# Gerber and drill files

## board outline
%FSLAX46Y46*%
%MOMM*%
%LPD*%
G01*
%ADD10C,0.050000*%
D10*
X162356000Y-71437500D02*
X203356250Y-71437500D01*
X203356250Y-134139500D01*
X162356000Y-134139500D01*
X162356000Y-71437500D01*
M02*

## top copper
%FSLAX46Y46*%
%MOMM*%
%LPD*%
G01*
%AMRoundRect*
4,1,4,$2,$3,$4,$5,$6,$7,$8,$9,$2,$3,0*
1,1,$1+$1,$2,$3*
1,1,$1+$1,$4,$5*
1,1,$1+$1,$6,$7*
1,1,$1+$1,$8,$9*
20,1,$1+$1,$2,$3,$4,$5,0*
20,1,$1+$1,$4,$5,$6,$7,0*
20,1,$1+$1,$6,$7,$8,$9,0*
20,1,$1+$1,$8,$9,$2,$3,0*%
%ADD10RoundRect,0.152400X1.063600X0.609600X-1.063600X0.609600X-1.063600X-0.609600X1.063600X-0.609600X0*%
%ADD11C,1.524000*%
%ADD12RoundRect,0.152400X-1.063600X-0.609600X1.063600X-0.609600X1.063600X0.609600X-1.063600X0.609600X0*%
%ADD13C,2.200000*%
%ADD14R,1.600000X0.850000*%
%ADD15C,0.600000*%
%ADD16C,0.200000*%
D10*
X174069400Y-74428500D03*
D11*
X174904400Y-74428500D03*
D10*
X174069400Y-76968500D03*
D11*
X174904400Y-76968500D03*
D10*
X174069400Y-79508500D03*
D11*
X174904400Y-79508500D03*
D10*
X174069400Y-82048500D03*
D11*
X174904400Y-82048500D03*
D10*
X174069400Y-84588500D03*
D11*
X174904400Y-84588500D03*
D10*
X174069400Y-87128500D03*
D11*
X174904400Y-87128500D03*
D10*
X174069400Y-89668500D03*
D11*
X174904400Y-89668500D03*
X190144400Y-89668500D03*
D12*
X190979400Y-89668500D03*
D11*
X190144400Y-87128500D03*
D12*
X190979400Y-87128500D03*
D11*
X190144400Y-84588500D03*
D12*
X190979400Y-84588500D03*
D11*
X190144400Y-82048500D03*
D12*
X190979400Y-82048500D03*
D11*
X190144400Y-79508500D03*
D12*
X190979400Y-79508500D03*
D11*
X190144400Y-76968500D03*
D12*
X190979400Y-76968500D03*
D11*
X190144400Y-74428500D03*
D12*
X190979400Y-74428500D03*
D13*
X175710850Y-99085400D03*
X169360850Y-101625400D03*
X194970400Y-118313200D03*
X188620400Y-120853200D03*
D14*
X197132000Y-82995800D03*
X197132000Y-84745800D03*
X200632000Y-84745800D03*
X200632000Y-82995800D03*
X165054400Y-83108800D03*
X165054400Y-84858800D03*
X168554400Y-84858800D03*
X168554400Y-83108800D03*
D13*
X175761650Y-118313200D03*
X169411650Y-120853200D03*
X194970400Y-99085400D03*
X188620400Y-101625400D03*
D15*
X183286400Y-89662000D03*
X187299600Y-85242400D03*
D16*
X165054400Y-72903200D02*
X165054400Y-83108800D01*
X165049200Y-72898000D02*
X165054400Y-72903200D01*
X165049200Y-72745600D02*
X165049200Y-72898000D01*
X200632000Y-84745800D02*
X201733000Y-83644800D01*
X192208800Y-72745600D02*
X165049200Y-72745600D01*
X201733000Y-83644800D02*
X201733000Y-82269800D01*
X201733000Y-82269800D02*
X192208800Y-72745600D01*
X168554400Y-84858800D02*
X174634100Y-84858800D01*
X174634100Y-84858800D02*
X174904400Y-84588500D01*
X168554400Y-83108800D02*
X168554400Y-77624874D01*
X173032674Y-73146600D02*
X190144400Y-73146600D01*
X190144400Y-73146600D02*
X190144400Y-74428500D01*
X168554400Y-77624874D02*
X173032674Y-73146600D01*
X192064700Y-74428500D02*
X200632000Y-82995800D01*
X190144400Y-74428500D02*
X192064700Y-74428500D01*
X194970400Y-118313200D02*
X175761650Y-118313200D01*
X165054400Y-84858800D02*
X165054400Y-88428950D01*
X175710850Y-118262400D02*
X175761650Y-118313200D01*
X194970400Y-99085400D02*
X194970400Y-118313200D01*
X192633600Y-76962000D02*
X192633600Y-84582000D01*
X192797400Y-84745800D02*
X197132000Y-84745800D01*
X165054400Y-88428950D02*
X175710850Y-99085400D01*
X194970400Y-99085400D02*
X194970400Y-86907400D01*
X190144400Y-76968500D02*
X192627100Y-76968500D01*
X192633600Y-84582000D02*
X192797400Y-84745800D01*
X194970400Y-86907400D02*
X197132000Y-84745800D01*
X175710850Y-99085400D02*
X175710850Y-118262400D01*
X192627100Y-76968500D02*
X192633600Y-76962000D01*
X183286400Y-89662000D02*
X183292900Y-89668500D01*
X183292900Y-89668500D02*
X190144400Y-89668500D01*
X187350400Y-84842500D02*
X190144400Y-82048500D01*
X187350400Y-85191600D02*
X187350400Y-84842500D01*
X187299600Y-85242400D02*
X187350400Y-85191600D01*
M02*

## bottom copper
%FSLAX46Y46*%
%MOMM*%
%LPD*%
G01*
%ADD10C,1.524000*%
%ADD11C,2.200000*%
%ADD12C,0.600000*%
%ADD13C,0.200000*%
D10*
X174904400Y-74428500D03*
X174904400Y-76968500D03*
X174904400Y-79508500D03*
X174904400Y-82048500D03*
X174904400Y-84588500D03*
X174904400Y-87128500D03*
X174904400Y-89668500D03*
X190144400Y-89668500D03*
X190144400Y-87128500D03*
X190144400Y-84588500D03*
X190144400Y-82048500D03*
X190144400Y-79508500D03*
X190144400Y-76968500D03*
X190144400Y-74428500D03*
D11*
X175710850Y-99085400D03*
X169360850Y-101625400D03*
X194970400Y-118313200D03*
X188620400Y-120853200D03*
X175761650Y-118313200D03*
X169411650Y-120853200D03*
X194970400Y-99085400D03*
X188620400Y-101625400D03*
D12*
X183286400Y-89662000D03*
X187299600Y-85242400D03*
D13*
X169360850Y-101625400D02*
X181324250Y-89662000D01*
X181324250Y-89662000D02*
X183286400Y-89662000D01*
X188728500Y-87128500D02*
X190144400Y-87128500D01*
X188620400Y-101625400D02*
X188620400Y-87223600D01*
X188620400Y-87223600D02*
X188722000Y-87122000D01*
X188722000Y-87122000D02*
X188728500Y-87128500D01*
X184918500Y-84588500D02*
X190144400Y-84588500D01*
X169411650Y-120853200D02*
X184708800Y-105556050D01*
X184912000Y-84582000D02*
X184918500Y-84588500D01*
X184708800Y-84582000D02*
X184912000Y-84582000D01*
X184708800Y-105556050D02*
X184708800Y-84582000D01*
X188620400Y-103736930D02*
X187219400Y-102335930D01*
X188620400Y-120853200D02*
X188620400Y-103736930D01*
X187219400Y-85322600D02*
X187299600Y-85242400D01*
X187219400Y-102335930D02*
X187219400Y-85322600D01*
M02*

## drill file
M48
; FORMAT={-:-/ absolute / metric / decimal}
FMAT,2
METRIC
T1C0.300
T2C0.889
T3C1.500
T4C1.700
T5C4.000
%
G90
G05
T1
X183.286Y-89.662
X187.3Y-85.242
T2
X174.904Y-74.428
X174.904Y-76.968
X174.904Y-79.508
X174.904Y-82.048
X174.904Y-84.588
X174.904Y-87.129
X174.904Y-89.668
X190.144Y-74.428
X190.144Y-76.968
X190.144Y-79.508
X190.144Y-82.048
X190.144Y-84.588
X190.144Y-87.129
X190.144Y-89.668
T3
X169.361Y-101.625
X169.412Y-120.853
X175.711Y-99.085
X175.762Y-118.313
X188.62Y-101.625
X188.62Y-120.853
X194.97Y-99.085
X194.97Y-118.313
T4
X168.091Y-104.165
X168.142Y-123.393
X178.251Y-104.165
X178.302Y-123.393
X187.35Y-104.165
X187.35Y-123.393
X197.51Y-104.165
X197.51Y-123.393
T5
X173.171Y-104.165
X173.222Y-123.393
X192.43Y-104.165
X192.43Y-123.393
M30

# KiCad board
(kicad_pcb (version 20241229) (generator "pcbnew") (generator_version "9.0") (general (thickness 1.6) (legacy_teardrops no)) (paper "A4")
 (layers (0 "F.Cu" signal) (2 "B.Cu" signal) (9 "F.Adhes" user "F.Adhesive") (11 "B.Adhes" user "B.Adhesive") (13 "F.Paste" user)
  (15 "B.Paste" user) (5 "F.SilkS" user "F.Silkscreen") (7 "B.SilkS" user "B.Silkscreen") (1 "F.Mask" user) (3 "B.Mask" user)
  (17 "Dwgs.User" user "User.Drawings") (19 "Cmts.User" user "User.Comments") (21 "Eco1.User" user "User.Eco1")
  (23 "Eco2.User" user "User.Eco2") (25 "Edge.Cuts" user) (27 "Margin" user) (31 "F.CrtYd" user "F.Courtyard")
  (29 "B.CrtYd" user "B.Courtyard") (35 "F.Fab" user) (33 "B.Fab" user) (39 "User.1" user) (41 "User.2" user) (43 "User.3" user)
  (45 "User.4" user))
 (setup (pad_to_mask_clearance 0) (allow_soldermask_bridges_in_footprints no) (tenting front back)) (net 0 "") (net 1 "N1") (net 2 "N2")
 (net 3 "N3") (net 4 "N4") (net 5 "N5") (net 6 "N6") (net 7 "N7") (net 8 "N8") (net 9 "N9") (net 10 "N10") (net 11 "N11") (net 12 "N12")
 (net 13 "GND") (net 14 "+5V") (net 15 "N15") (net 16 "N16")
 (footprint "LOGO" (layer "F.Cu") (at 199.6948 74.5236)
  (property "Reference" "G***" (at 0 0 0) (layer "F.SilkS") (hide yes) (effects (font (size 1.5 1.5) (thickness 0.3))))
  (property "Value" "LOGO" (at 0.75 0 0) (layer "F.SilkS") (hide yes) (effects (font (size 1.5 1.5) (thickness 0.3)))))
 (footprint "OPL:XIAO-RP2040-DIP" (layer "F.Cu") (at 182.5244 82.0485)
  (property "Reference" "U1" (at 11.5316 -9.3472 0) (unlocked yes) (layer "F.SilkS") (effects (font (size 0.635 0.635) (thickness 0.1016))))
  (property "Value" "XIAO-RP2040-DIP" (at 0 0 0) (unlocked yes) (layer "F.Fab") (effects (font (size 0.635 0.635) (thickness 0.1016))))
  (pad "1" smd roundrect (at -8.455 -7.62 180) (size 2.432 1.524) (layers "F.Cu" "F.Mask") (roundrect_rratio 0.1) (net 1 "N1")
   (thermal_bridge_angle 45))
  (pad "1" thru_hole circle (at -7.62 -7.62 180) (size 1.524 1.524) (drill 0.889) (layers "*.Cu" "*.Mask") (remove_unused_layers no)
   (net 1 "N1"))
  (pad "2" smd roundrect (at -8.455 -5.08 180) (size 2.432 1.524) (layers "F.Cu" "F.Mask") (roundrect_rratio 0.1) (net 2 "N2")
   (thermal_bridge_angle 45))
  (pad "2" thru_hole circle (at -7.62 -5.08 180) (size 1.524 1.524) (drill 0.889) (layers "*.Cu" "*.Mask") (remove_unused_layers no)
   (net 2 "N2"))
  (pad "3" smd roundrect (at -8.455 -2.54 180) (size 2.432 1.524) (layers "F.Cu" "F.Mask") (roundrect_rratio 0.1) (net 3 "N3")
   (thermal_bridge_angle 45))
  (pad "3" thru_hole circle (at -7.62 -2.54 180) (size 1.524 1.524) (drill 0.889) (layers "*.Cu" "*.Mask") (remove_unused_layers no)
   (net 3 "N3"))
  (pad "4" smd roundrect (at -8.455 0 180) (size 2.432 1.524) (layers "F.Cu" "F.Mask") (roundrect_rratio 0.1) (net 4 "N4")
   (thermal_bridge_angle 45))
  (pad "4" thru_hole circle (at -7.62 0 180) (size 1.524 1.524) (drill 0.889) (layers "*.Cu" "*.Mask") (remove_unused_layers no)
   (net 4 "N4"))
  (pad "5" smd roundrect (at -8.455 2.54 180) (size 2.432 1.524) (layers "F.Cu" "F.Mask") (roundrect_rratio 0.1) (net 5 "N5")
   (thermal_bridge_angle 45))
  (pad "5" thru_hole circle (at -7.62 2.54 180) (size 1.524 1.524) (drill 0.889) (layers "*.Cu" "*.Mask") (remove_unused_layers no)
   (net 5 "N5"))
  (pad "6" smd roundrect (at -8.455 5.08 180) (size 2.432 1.524) (layers "F.Cu" "F.Mask") (roundrect_rratio 0.1) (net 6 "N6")
   (thermal_bridge_angle 45))
  (pad "6" thru_hole circle (at -7.62 5.08 180) (size 1.524 1.524) (drill 0.889) (layers "*.Cu" "*.Mask") (remove_unused_layers no)
   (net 6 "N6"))
  (pad "7" smd roundrect (at -8.455 7.62 180) (size 2.432 1.524) (layers "F.Cu" "F.Mask") (roundrect_rratio 0.1) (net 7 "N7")
   (thermal_bridge_angle 45))
  (pad "7" thru_hole circle (at -7.62 7.62 180) (size 1.524 1.524) (drill 0.889) (layers "*.Cu" "*.Mask") (remove_unused_layers no)
   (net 7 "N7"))
  (pad "8" thru_hole circle (at 7.62 7.62) (size 1.524 1.524) (drill 0.889) (layers "*.Cu" "*.Mask") (remove_unused_layers no) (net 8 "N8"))
  (pad "8" smd roundrect (at 8.455 7.62) (size 2.432 1.524) (layers "F.Cu" "F.Mask") (roundrect_rratio 0.1) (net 8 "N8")
   (thermal_bridge_angle 45))
  (pad "9" thru_hole circle (at 7.62 5.08) (size 1.524 1.524) (drill 0.889) (layers "*.Cu" "*.Mask") (remove_unused_layers no) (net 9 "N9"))
  (pad "9" smd roundrect (at 8.455 5.08) (size 2.432 1.524) (layers "F.Cu" "F.Mask") (roundrect_rratio 0.1) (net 9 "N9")
   (thermal_bridge_angle 45))
  (pad "10" thru_hole circle (at 7.62 2.54) (size 1.524 1.524) (drill 0.889) (layers "*.Cu" "*.Mask") (remove_unused_layers no)
   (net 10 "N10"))
  (pad "10" smd roundrect (at 8.455 2.54) (size 2.432 1.524) (layers "F.Cu" "F.Mask") (roundrect_rratio 0.1) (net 10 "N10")
   (thermal_bridge_angle 45))
  (pad "11" thru_hole circle (at 7.62 0) (size 1.524 1.524) (drill 0.889) (layers "*.Cu" "*.Mask") (remove_unused_layers no) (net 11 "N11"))
  (pad "11" smd roundrect (at 8.455 0) (size 2.432 1.524) (layers "F.Cu" "F.Mask") (roundrect_rratio 0.1) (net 11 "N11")
   (thermal_bridge_angle 45))
  (pad "12" thru_hole circle (at 7.62 -2.54) (size 1.524 1.524) (drill 0.889) (layers "*.Cu" "*.Mask") (remove_unused_layers no)
   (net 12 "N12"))
  (pad "12" smd roundrect (at 8.455 -2.54) (size 2.432 1.524) (layers "F.Cu" "F.Mask") (roundrect_rratio 0.1) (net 12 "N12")
   (thermal_bridge_angle 45))
  (pad "13" thru_hole circle (at 7.62 -5.08) (size 1.524 1.524) (drill 0.889) (layers "*.Cu" "*.Mask") (remove_unused_layers no)
   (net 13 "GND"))
  (pad "13" smd roundrect (at 8.455 -5.08) (size 2.432 1.524) (layers "F.Cu" "F.Mask") (roundrect_rratio 0.1) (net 13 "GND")
   (thermal_bridge_angle 45))
  (pad "14" thru_hole circle (at 7.62 -7.62) (size 1.524 1.524) (drill 0.889) (layers "*.Cu" "*.Mask") (remove_unused_layers no)
   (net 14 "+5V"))
  (pad "14" smd roundrect (at 8.455 -7.62) (size 2.432 1.524) (layers "F.Cu" "F.Mask") (roundrect_rratio 0.1) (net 14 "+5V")
   (thermal_bridge_angle 45)))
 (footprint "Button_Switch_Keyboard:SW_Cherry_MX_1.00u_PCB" (layer "F.Cu") (at 175.71085 99.0854)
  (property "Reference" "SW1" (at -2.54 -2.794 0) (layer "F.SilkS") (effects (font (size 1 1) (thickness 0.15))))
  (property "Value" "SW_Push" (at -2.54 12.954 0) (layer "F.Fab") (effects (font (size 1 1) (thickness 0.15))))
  (pad "" np_thru_hole circle (at -7.62 5.08) (size 1.7 1.7) (drill 1.7) (layers "*.Cu" "*.Mask"))
  (pad "" np_thru_hole circle (at -2.54 5.08) (size 4 4) (drill 4) (layers "*.Cu" "*.Mask"))
  (pad "" np_thru_hole circle (at 2.54 5.08) (size 1.7 1.7) (drill 1.7) (layers "*.Cu" "*.Mask"))
  (pad "1" thru_hole circle (at 0 0) (size 2.2 2.2) (drill 1.5) (layers "*.Cu" "*.Mask") (remove_unused_layers no) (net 13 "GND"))
  (pad "2" thru_hole circle (at -6.35 2.54) (size 2.2 2.2) (drill 1.5) (layers "*.Cu" "*.Mask") (remove_unused_layers no) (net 8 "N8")))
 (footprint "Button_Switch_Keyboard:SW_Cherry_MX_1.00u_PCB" (layer "F.Cu") (at 194.9704 118.3132)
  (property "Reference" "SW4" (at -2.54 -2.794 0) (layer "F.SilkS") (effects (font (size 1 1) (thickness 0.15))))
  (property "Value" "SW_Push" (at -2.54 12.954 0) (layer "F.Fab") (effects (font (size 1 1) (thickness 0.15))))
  (pad "" np_thru_hole circle (at -7.62 5.08) (size 1.7 1.7) (drill 1.7) (layers "*.Cu" "*.Mask"))
  (pad "" np_thru_hole circle (at -2.54 5.08) (size 4 4) (drill 4) (layers "*.Cu" "*.Mask"))
  (pad "" np_thru_hole circle (at 2.54 5.08) (size 1.7 1.7) (drill 1.7) (layers "*.Cu" "*.Mask"))
  (pad "1" thru_hole circle (at 0 0) (size 2.2 2.2) (drill 1.5) (layers "*.Cu" "*.Mask") (remove_unused_layers no) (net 13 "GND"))
  (pad "2" thru_hole circle (at -6.35 2.54) (size 2.2 2.2) (drill 1.5) (layers "*.Cu" "*.Mask") (remove_unused_layers no) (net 11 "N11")))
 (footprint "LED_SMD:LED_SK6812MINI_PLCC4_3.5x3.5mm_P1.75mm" (layer "F.Cu") (at 198.882 83.8708)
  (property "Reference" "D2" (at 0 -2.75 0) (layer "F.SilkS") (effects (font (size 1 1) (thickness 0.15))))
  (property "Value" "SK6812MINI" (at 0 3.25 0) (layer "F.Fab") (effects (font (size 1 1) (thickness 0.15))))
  (pad "1" smd rect (at -1.75 -0.875) (size 1.6 0.85) (layers "F.Cu" "F.Mask" "F.Paste") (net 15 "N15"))
  (pad "2" smd rect (at -1.75 0.875) (size 1.6 0.85) (layers "F.Cu" "F.Mask" "F.Paste") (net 13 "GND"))
  (pad "3" smd rect (at 1.75 0.875) (size 1.6 0.85) (layers "F.Cu" "F.Mask" "F.Paste") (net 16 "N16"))
  (pad "4" smd rect (at 1.75 -0.875) (size 1.6 0.85) (layers "F.Cu" "F.Mask" "F.Paste") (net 14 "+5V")))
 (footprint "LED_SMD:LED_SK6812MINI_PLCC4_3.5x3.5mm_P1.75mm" (layer "F.Cu") (at 166.8044 83.9838)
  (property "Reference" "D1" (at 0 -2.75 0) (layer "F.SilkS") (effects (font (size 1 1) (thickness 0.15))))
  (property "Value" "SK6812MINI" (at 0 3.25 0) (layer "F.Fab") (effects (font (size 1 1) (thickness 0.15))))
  (pad "1" smd rect (at -1.75 -0.875) (size 1.6 0.85) (layers "F.Cu" "F.Mask" "F.Paste") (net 16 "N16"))
  (pad "2" smd rect (at -1.75 0.875) (size 1.6 0.85) (layers "F.Cu" "F.Mask" "F.Paste") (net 13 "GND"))
  (pad "3" smd rect (at 1.75 0.875) (size 1.6 0.85) (layers "F.Cu" "F.Mask" "F.Paste") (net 5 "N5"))
  (pad "4" smd rect (at 1.75 -0.875) (size 1.6 0.85) (layers "F.Cu" "F.Mask" "F.Paste") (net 14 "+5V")))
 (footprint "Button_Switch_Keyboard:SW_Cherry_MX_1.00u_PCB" (layer "F.Cu") (at 175.76165 118.3132)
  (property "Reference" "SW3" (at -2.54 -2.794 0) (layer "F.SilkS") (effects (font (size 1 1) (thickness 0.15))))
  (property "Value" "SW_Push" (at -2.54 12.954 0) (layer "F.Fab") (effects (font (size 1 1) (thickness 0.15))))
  (pad "" np_thru_hole circle (at -7.62 5.08) (size 1.7 1.7) (drill 1.7) (layers "*.Cu" "*.Mask"))
  (pad "" np_thru_hole circle (at -2.54 5.08) (size 4 4) (drill 4) (layers "*.Cu" "*.Mask"))
  (pad "" np_thru_hole circle (at 2.54 5.08) (size 1.7 1.7) (drill 1.7) (layers "*.Cu" "*.Mask"))
  (pad "1" thru_hole circle (at 0 0) (size 2.2 2.2) (drill 1.5) (layers "*.Cu" "*.Mask") (remove_unused_layers no) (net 13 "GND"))
  (pad "2" thru_hole circle (at -6.35 2.54) (size 2.2 2.2) (drill 1.5) (layers "*.Cu" "*.Mask") (remove_unused_layers no) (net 10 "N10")))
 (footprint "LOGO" (layer "F.Cu") (at 165.9128 74.3204)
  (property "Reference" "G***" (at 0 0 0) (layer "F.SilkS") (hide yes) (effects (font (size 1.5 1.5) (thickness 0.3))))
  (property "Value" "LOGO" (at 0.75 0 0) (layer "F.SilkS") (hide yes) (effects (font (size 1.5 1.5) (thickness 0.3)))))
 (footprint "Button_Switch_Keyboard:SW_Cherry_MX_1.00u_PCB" (layer "F.Cu") (at 194.9704 99.0854)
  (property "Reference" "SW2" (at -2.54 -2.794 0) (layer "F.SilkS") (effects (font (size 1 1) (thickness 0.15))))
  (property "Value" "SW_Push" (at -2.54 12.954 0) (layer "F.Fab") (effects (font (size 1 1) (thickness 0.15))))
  (pad "" np_thru_hole circle (at -7.62 5.08) (size 1.7 1.7) (drill 1.7) (layers "*.Cu" "*.Mask"))
  (pad "" np_thru_hole circle (at -2.54 5.08) (size 4 4) (drill 4) (layers "*.Cu" "*.Mask"))
  (pad "" np_thru_hole circle (at 2.54 5.08) (size 1.7 1.7) (drill 1.7) (layers "*.Cu" "*.Mask"))
  (pad "1" thru_hole circle (at 0 0) (size 2.2 2.2) (drill 1.5) (layers "*.Cu" "*.Mask") (remove_unused_layers no) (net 13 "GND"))
  (pad "2" thru_hole circle (at -6.35 2.54) (size 2.2 2.2) (drill 1.5) (layers "*.Cu" "*.Mask") (remove_unused_layers no) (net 9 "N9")))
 (gr_rect (start 162.356 71.4375) (end 203.35625 134.1395) (stroke (width 0.05) (type solid)) (fill no) (layer "Edge.Cuts"))
 (segment (start 165.0544 72.9032) (end 165.0544 83.1088) (width 0.2) (layer "F.Cu") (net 16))
 (segment (start 165.0492 72.898) (end 165.0544 72.9032) (width 0.2) (layer "F.Cu") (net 16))
 (segment (start 165.0492 72.7456) (end 165.0492 72.898) (width 0.2) (layer "F.Cu") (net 16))
 (segment (start 200.632 84.7458) (end 201.733 83.6448) (width 0.2) (layer "F.Cu") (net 16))
 (segment (start 192.2088 72.7456) (end 165.0492 72.7456) (width 0.2) (layer "F.Cu") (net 16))
 (segment (start 201.733 83.6448) (end 201.733 82.2698) (width 0.2) (layer "F.Cu") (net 16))
 (segment (start 201.733 82.2698) (end 192.2088 72.7456) (width 0.2) (layer "F.Cu") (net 16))
 (segment (start 168.5544 84.8588) (end 174.6341 84.8588) (width 0.2) (layer "F.Cu") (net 5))
 (segment (start 174.6341 84.8588) (end 174.9044 84.5885) (width 0.2) (layer "F.Cu") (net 5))
 (segment (start 168.5544 83.1088) (end 168.5544 77.624874) (width 0.2) (layer "F.Cu") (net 14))
 (segment (start 173.032674 73.1466) (end 190.1444 73.1466) (width 0.2) (layer "F.Cu") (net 14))
 (segment (start 190.1444 73.1466) (end 190.1444 74.4285) (width 0.2) (layer "F.Cu") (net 14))
 (segment (start 168.5544 77.624874) (end 173.032674 73.1466) (width 0.2) (layer "F.Cu") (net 14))
 (segment (start 192.0647 74.4285) (end 200.632 82.9958) (width 0.2) (layer "F.Cu") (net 14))
 (segment (start 190.1444 74.4285) (end 192.0647 74.4285) (width 0.2) (layer "F.Cu") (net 14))
 (segment (start 194.9704 118.3132) (end 175.76165 118.3132) (width 0.2) (layer "F.Cu") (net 13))
 (segment (start 165.0544 84.8588) (end 165.0544 88.42895) (width 0.2) (layer "F.Cu") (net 13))
 (segment (start 175.71085 118.2624) (end 175.76165 118.3132) (width 0.2) (layer "F.Cu") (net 13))
 (segment (start 194.9704 99.0854) (end 194.9704 118.3132) (width 0.2) (layer "F.Cu") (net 13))
 (segment (start 192.6336 76.962) (end 192.6336 84.582) (width 0.2) (layer "F.Cu") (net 13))
 (segment (start 192.7974 84.7458) (end 197.132 84.7458) (width 0.2) (layer "F.Cu") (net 13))
 (segment (start 165.0544 88.42895) (end 175.71085 99.0854) (width 0.2) (layer "F.Cu") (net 13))
 (segment (start 194.9704 99.0854) (end 194.9704 86.9074) (width 0.2) (layer "F.Cu") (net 13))
 (segment (start 190.1444 76.9685) (end 192.6271 76.9685) (width 0.2) (layer "F.Cu") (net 13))
 (segment (start 192.6336 84.582) (end 192.7974 84.7458) (width 0.2) (layer "F.Cu") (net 13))
 (segment (start 194.9704 86.9074) (end 197.132 84.7458) (width 0.2) (layer "F.Cu") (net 13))
 (segment (start 175.71085 99.0854) (end 175.71085 118.2624) (width 0.2) (layer "F.Cu") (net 13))
 (segment (start 192.6271 76.9685) (end 192.6336 76.962) (width 0.2) (layer "F.Cu") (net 13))
 (segment (start 183.2864 89.662) (end 183.2929 89.6685) (width 0.2) (layer "F.Cu") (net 8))
 (segment (start 183.2929 89.6685) (end 190.1444 89.6685) (width 0.2) (layer "F.Cu") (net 8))
 (via (at 183.2864 89.662) (size 0.6) (drill 0.3) (layers "F.Cu" "B.Cu") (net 8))
 (segment (start 169.36085 101.6254) (end 181.32425 89.662) (width 0.2) (layer "B.Cu") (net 8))
 (segment (start 181.32425 89.662) (end 183.2864 89.662) (width 0.2) (layer "B.Cu") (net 8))
 (segment (start 188.7285 87.1285) (end 190.1444 87.1285) (width 0.2) (layer "B.Cu") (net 9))
 (segment (start 188.6204 101.6254) (end 188.6204 87.2236) (width 0.2) (layer "B.Cu") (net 9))
 (segment (start 188.6204 87.2236) (end 188.722 87.122) (width 0.2) (layer "B.Cu") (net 9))
 (segment (start 188.722 87.122) (end 188.7285 87.1285) (width 0.2) (layer "B.Cu") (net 9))
 (segment (start 184.9185 84.5885) (end 190.1444 84.5885) (width 0.2) (layer "B.Cu") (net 10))
 (segment (start 169.41165 120.8532) (end 184.7088 105.55605) (width 0.2) (layer "B.Cu") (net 10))
 (segment (start 184.912 84.582) (end 184.9185 84.5885) (width 0.2) (layer "B.Cu") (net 10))
 (segment (start 184.7088 84.582) (end 184.912 84.582) (width 0.2) (layer "B.Cu") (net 10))
 (segment (start 184.7088 105.55605) (end 184.7088 84.582) (width 0.2) (layer "B.Cu") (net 10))
 (segment (start 187.3504 84.8425) (end 190.1444 82.0485) (width 0.2) (layer "F.Cu") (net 11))
 (segment (start 187.3504 85.1916) (end 187.3504 84.8425) (width 0.2) (layer "F.Cu") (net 11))
 (segment (start 187.2996 85.2424) (end 187.3504 85.1916) (width 0.2) (layer "F.Cu") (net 11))
 (via (at 187.2996 85.2424) (size 0.6) (drill 0.3) (layers "F.Cu" "B.Cu") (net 11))
 (segment (start 188.6204 103.73693) (end 187.2194 102.33593) (width 0.2) (layer "B.Cu") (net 11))
 (segment (start 188.6204 120.8532) (end 188.6204 103.73693) (width 0.2) (layer "B.Cu") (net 11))
 (segment (start 187.2194 85.3226) (end 187.2996 85.2424) (width 0.2) (layer "B.Cu") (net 11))
 (segment (start 187.2194 102.33593) (end 187.2194 85.3226) (width 0.2) (layer "B.Cu") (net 11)))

